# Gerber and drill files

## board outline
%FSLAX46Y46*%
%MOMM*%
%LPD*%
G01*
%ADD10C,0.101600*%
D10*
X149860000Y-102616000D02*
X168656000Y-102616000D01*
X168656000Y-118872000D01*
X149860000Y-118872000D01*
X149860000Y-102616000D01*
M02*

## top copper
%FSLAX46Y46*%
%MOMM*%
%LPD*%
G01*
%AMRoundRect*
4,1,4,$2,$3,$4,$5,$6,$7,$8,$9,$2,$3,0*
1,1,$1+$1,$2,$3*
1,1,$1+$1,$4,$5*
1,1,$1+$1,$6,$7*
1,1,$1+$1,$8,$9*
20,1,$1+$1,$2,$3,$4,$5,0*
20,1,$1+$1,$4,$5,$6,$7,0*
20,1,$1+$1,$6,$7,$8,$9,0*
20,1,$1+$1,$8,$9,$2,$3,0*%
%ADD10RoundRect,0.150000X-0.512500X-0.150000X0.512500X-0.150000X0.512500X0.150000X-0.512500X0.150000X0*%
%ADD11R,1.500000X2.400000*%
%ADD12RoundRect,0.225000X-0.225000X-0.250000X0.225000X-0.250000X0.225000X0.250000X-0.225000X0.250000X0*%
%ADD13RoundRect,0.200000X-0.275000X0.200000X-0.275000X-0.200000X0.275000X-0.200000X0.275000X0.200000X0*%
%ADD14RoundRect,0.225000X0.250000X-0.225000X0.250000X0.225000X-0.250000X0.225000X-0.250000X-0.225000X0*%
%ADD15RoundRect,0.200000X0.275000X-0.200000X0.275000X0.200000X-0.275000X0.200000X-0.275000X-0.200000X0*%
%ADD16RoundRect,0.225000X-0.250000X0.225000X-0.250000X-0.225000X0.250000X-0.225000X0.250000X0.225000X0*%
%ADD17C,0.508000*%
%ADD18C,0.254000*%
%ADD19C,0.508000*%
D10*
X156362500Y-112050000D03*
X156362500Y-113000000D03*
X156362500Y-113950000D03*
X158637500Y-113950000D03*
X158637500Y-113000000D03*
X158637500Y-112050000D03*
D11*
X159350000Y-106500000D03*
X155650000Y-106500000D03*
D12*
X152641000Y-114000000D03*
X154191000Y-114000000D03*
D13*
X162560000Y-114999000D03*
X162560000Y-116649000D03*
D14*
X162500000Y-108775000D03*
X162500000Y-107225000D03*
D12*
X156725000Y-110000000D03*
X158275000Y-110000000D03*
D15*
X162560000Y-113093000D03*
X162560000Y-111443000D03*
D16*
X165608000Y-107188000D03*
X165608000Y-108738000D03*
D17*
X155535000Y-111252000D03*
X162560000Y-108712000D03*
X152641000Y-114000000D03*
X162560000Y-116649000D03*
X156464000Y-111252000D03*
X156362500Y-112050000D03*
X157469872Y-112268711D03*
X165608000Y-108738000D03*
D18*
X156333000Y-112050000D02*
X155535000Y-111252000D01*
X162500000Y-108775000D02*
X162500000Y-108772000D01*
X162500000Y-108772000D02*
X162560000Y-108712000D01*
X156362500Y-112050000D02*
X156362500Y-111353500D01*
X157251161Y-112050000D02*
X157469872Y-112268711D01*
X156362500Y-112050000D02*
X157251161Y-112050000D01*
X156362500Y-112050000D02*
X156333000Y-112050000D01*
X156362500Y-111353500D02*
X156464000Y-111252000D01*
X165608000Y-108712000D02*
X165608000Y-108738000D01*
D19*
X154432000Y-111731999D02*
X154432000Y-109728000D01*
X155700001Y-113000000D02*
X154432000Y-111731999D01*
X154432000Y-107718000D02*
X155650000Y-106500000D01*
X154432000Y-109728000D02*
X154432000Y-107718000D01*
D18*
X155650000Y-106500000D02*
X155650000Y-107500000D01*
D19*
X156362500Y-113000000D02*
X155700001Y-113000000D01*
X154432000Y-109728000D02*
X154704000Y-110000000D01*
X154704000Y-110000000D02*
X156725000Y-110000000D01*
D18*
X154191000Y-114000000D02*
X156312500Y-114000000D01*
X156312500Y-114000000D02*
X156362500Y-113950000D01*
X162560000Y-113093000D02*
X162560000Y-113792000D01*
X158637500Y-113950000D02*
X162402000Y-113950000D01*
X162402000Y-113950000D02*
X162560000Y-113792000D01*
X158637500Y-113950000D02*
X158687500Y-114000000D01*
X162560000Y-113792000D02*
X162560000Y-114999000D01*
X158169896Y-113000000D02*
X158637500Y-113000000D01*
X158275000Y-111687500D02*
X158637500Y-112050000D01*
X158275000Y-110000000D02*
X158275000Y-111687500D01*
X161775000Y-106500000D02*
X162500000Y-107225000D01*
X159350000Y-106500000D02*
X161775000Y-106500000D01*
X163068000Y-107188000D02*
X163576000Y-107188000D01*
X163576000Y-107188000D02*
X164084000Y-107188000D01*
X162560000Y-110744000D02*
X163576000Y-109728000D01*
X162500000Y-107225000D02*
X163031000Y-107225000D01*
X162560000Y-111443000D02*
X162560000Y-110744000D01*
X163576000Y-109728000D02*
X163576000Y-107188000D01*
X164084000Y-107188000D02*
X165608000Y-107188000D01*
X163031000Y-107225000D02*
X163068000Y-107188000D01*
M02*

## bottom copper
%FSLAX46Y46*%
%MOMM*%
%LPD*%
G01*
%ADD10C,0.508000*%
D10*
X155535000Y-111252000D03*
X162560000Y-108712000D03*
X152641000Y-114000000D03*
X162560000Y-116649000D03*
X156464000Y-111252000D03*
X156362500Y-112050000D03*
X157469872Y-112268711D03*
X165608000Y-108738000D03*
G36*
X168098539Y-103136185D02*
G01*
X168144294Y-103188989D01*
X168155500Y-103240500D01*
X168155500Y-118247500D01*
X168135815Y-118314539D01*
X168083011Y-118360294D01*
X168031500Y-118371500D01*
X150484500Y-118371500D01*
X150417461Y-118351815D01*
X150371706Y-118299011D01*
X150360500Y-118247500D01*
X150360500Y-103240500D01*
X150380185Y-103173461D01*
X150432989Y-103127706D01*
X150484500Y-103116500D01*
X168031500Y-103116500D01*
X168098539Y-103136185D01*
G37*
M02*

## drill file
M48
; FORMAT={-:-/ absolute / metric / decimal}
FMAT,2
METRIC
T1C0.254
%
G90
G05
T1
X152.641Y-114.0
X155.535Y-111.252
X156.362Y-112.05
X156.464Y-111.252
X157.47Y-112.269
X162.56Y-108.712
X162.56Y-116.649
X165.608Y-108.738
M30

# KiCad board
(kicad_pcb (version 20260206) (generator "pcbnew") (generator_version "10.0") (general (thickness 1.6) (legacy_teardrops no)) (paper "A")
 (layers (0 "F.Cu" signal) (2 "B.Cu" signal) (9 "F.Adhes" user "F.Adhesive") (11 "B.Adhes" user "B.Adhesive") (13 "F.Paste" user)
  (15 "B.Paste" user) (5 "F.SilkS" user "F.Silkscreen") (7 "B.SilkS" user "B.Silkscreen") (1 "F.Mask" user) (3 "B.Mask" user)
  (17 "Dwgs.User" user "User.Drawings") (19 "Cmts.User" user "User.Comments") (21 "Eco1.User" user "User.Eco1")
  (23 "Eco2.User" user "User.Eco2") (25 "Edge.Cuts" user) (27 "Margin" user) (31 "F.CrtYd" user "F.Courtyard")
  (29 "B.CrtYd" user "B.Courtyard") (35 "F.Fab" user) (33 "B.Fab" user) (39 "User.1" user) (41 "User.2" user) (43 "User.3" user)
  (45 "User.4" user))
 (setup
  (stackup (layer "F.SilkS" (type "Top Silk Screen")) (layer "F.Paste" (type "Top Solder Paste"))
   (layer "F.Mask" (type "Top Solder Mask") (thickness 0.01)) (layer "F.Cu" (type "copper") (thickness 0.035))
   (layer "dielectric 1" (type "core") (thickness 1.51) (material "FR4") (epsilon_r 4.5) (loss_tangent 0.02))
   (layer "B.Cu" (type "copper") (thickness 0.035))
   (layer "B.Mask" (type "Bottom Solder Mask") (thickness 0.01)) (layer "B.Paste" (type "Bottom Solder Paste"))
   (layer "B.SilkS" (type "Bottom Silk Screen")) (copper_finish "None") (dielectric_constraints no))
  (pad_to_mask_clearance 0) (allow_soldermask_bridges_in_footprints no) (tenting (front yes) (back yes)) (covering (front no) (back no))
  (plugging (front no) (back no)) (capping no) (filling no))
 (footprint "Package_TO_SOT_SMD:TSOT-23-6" (layer "F.Cu") (at 157.5 113)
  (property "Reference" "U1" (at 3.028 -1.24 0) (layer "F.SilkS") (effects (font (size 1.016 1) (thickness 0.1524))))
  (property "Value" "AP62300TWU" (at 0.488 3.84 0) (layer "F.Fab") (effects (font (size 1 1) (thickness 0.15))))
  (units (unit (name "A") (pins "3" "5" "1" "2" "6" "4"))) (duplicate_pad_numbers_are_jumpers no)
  (pad "1" smd roundrect (at -1.1375 -0.95) (size 1.325 0.6) (layers "F.Cu" "F.Mask" "F.Paste") (roundrect_rratio 0.25) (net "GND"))
  (pad "2" smd roundrect (at -1.1375 0) (size 1.325 0.6) (layers "F.Cu" "F.Mask" "F.Paste") (roundrect_rratio 0.25) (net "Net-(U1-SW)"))
  (pad "3" smd roundrect (at -1.1375 0.95) (size 1.325 0.6) (layers "F.Cu" "F.Mask" "F.Paste") (roundrect_rratio 0.25) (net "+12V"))
  (pad "4" smd roundrect (at 1.1375 0.95) (size 1.325 0.6) (layers "F.Cu" "F.Mask" "F.Paste") (roundrect_rratio 0.25) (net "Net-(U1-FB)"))
  (pad "5" smd roundrect (at 1.1375 0) (size 1.325 0.6) (layers "F.Cu" "F.Mask" "F.Paste") (roundrect_rratio 0.25)
   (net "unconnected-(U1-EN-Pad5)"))
  (pad "6" smd roundrect (at 1.1375 -0.95) (size 1.325 0.6) (layers "F.Cu" "F.Mask" "F.Paste") (roundrect_rratio 0.25) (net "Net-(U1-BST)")))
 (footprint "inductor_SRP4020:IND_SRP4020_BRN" (layer "F.Cu") (at 157.5 106.5 180)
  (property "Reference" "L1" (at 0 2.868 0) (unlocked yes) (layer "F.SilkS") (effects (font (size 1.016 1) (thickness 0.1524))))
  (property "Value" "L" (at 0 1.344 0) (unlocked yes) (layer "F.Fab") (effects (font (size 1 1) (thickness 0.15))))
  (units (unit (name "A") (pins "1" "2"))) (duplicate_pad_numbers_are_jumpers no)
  (pad "1" smd rect (at -1.85 0 270) (size 2.4 1.5) (layers "F.Cu" "F.Mask" "F.Paste") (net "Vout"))
  (pad "2" smd rect (at 1.85 0 270) (size 2.4 1.5) (layers "F.Cu" "F.Mask" "F.Paste") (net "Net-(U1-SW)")))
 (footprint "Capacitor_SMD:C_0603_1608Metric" (layer "F.Cu") (at 153.416 114)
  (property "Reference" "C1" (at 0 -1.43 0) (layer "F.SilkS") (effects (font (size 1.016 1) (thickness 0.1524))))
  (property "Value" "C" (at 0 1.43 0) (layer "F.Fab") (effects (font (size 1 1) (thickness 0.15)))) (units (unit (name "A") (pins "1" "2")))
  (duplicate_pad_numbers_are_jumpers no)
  (pad "1" smd roundrect (at -0.775 0) (size 0.9 0.95) (layers "F.Cu" "F.Mask" "F.Paste") (roundrect_rratio 0.25) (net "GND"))
  (pad "2" smd roundrect (at 0.775 0) (size 0.9 0.95) (layers "F.Cu" "F.Mask" "F.Paste") (roundrect_rratio 0.25) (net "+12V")))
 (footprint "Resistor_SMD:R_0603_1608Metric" (layer "F.Cu") (at 162.56 115.824 -90)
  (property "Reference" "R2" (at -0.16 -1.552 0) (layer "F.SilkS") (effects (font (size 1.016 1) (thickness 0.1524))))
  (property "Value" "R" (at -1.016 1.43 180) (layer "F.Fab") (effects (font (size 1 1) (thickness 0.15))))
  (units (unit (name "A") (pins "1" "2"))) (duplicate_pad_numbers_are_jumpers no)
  (pad "1" smd roundrect (at -0.825 0 270) (size 0.8 0.95) (layers "F.Cu" "F.Mask" "F.Paste") (roundrect_rratio 0.25) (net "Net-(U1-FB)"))
  (pad "2" smd roundrect (at 0.825 0 270) (size 0.8 0.95) (layers "F.Cu" "F.Mask" "F.Paste") (roundrect_rratio 0.25) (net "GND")))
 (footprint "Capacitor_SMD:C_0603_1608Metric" (layer "F.Cu") (at 162.5 108 90)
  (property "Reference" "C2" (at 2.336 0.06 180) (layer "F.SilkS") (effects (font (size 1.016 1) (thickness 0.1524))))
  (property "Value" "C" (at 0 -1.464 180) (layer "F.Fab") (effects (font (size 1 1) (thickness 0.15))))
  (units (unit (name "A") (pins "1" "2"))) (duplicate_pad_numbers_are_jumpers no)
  (pad "1" smd roundrect (at -0.775 0 90) (size 0.9 0.95) (layers "F.Cu" "F.Mask" "F.Paste") (roundrect_rratio 0.25) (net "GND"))
  (pad "2" smd roundrect (at 0.775 0 90) (size 0.9 0.95) (layers "F.Cu" "F.Mask" "F.Paste") (roundrect_rratio 0.25) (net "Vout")))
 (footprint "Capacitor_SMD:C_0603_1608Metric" (layer "F.Cu") (at 157.5 110)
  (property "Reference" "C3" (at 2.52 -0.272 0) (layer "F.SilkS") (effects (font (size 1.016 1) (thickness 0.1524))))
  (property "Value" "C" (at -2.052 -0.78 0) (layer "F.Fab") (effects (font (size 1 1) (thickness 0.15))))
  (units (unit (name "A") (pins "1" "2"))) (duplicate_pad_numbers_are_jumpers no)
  (pad "1" smd roundrect (at -0.775 0) (size 0.9 0.95) (layers "F.Cu" "F.Mask" "F.Paste") (roundrect_rratio 0.25) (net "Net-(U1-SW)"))
  (pad "2" smd roundrect (at 0.775 0) (size 0.9 0.95) (layers "F.Cu" "F.Mask" "F.Paste") (roundrect_rratio 0.25) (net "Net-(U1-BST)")))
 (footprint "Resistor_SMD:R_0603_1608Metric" (layer "F.Cu") (at 162.56 112.268 90)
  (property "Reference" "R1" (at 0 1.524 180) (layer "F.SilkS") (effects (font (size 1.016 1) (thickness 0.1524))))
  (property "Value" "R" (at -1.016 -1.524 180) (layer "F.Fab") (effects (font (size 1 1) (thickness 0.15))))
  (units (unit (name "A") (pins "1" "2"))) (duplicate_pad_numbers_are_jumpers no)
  (pad "1" smd roundrect (at -0.825 0 90) (size 0.8 0.95) (layers "F.Cu" "F.Mask" "F.Paste") (roundrect_rratio 0.25) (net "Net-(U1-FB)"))
  (pad "2" smd roundrect (at 0.825 0 90) (size 0.8 0.95) (layers "F.Cu" "F.Mask" "F.Paste") (roundrect_rratio 0.25) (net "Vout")))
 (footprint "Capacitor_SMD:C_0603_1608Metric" (layer "F.Cu") (at 165.608 107.963 -90)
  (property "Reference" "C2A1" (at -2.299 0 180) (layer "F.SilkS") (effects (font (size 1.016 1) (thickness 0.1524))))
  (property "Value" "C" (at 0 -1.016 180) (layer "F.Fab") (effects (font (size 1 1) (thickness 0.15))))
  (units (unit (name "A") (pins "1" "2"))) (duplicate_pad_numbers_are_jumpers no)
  (pad "1" smd roundrect (at -0.775 0 270) (size 0.9 0.95) (layers "F.Cu" "F.Mask" "F.Paste") (roundrect_rratio 0.25) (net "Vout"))
  (pad "2" smd roundrect (at 0.775 0 270) (size 0.9 0.95) (layers "F.Cu" "F.Mask" "F.Paste") (roundrect_rratio 0.25) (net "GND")))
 (gr_rect (start 149.86 102.616) (end 168.656 118.872) (stroke (width 0.1016) (type default)) (fill no) (layer "Edge.Cuts"))
 (segment (start 156.333 112.05) (end 155.535 111.252) (width 0.254) (layer "F.Cu") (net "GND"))
 (segment (start 162.5 108.775) (end 162.5 108.772) (width 0.254) (layer "F.Cu") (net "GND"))
 (segment (start 162.5 108.772) (end 162.56 108.712) (width 0.254) (layer "F.Cu") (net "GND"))
 (segment (start 156.3625 112.05) (end 156.3625 111.3535) (width 0.254) (layer "F.Cu") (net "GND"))
 (segment (start 157.251161 112.05) (end 157.469872 112.268711) (width 0.254) (layer "F.Cu") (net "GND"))
 (segment (start 156.3625 112.05) (end 157.251161 112.05) (width 0.254) (layer "F.Cu") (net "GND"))
 (segment (start 156.3625 112.05) (end 156.333 112.05) (width 0.254) (layer "F.Cu") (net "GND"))
 (segment (start 156.3625 111.3535) (end 156.464 111.252) (width 0.254) (layer "F.Cu") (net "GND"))
 (segment (start 165.608 108.712) (end 165.608 108.738) (width 0.254) (layer "F.Cu") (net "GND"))
 (via (at 155.535 111.252) (size 0.508) (drill 0.254) (layers "F.Cu" "B.Cu") (free yes) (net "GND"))
 (via (at 162.56 108.712) (size 0.508) (drill 0.254) (layers "F.Cu" "B.Cu") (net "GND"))
 (via (at 152.641 114) (size 0.508) (drill 0.254) (layers "F.Cu" "B.Cu") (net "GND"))
 (via (at 162.56 116.649) (size 0.508) (drill 0.254) (layers "F.Cu" "B.Cu") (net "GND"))
 (via (at 156.464 111.252) (size 0.508) (drill 0.254) (layers "F.Cu" "B.Cu") (free yes) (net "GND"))
 (via (at 156.3625 112.05) (size 0.508) (drill 0.254) (layers "F.Cu" "B.Cu") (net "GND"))
 (via (at 157.469872 112.268711) (size 0.508) (drill 0.254) (layers "F.Cu" "B.Cu") (free yes) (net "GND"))
 (via (at 165.608 108.738) (size 0.508) (drill 0.254) (layers "F.Cu" "B.Cu") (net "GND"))
 (segment (start 154.432 111.731999) (end 154.432 109.728) (width 0.508) (layer "F.Cu") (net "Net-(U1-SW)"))
 (segment (start 155.700001 113) (end 154.432 111.731999) (width 0.508) (layer "F.Cu") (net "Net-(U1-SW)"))
 (segment (start 154.432 107.718) (end 155.65 106.5) (width 0.508) (layer "F.Cu") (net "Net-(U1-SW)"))
 (segment (start 154.432 109.728) (end 154.432 107.718) (width 0.508) (layer "F.Cu") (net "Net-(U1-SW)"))
 (segment (start 155.65 106.5) (end 155.65 107.5) (width 0.254) (layer "F.Cu") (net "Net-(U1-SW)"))
 (segment (start 156.3625 113) (end 155.700001 113) (width 0.508) (layer "F.Cu") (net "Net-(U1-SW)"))
 (segment (start 154.432 109.728) (end 154.704 110) (width 0.508) (layer "F.Cu") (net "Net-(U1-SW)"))
 (segment (start 154.704 110) (end 156.725 110) (width 0.508) (layer "F.Cu") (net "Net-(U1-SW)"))
 (segment (start 154.191 114) (end 156.3125 114) (width 0.254) (layer "F.Cu") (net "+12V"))
 (segment (start 156.3125 114) (end 156.3625 113.95) (width 0.254) (layer "F.Cu") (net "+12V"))
 (segment (start 162.56 113.093) (end 162.56 113.792) (width 0.254) (layer "F.Cu") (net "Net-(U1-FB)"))
 (segment (start 158.6375 113.95) (end 162.402 113.95) (width 0.254) (layer "F.Cu") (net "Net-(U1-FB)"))
 (segment (start 162.402 113.95) (end 162.56 113.792) (width 0.254) (layer "F.Cu") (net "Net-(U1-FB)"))
 (segment (start 158.6375 113.95) (end 158.6875 114) (width 0.254) (layer "F.Cu") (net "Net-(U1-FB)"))
 (segment (start 162.56 113.792) (end 162.56 114.999) (width 0.254) (layer "F.Cu") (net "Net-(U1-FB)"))
 (segment (start 158.169896 113) (end 158.6375 113) (width 0.254) (layer "F.Cu") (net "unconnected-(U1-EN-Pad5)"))
 (segment (start 158.275 111.6875) (end 158.6375 112.05) (width 0.254) (layer "F.Cu") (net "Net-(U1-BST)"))
 (segment (start 158.275 110) (end 158.275 111.6875) (width 0.254) (layer "F.Cu") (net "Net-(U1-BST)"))
 (segment (start 161.775 106.5) (end 162.5 107.225) (width 0.254) (layer "F.Cu") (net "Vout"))
 (segment (start 159.35 106.5) (end 161.775 106.5) (width 0.254) (layer "F.Cu") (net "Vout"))
 (segment (start 163.068 107.188) (end 163.576 107.188) (width 0.254) (layer "F.Cu") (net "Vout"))
 (segment (start 163.576 107.188) (end 164.084 107.188) (width 0.254) (layer "F.Cu") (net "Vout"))
 (segment (start 162.56 110.744) (end 163.576 109.728) (width 0.254) (layer "F.Cu") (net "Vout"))
 (segment (start 162.5 107.225) (end 163.031 107.225) (width 0.254) (layer "F.Cu") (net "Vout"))
 (segment (start 162.56 111.443) (end 162.56 110.744) (width 0.254) (layer "F.Cu") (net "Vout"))
 (segment (start 163.576 109.728) (end 163.576 107.188) (width 0.254) (layer "F.Cu") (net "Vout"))
 (segment (start 164.084 107.188) (end 165.608 107.188) (width 0.254) (layer "F.Cu") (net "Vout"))
 (segment (start 163.031 107.225) (end 163.068 107.188) (width 0.254) (layer "F.Cu") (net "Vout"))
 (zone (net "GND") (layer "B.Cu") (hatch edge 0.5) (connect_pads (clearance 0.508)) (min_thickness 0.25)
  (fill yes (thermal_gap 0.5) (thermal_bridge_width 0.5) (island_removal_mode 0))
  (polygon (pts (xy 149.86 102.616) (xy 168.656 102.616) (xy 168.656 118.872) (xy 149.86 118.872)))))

